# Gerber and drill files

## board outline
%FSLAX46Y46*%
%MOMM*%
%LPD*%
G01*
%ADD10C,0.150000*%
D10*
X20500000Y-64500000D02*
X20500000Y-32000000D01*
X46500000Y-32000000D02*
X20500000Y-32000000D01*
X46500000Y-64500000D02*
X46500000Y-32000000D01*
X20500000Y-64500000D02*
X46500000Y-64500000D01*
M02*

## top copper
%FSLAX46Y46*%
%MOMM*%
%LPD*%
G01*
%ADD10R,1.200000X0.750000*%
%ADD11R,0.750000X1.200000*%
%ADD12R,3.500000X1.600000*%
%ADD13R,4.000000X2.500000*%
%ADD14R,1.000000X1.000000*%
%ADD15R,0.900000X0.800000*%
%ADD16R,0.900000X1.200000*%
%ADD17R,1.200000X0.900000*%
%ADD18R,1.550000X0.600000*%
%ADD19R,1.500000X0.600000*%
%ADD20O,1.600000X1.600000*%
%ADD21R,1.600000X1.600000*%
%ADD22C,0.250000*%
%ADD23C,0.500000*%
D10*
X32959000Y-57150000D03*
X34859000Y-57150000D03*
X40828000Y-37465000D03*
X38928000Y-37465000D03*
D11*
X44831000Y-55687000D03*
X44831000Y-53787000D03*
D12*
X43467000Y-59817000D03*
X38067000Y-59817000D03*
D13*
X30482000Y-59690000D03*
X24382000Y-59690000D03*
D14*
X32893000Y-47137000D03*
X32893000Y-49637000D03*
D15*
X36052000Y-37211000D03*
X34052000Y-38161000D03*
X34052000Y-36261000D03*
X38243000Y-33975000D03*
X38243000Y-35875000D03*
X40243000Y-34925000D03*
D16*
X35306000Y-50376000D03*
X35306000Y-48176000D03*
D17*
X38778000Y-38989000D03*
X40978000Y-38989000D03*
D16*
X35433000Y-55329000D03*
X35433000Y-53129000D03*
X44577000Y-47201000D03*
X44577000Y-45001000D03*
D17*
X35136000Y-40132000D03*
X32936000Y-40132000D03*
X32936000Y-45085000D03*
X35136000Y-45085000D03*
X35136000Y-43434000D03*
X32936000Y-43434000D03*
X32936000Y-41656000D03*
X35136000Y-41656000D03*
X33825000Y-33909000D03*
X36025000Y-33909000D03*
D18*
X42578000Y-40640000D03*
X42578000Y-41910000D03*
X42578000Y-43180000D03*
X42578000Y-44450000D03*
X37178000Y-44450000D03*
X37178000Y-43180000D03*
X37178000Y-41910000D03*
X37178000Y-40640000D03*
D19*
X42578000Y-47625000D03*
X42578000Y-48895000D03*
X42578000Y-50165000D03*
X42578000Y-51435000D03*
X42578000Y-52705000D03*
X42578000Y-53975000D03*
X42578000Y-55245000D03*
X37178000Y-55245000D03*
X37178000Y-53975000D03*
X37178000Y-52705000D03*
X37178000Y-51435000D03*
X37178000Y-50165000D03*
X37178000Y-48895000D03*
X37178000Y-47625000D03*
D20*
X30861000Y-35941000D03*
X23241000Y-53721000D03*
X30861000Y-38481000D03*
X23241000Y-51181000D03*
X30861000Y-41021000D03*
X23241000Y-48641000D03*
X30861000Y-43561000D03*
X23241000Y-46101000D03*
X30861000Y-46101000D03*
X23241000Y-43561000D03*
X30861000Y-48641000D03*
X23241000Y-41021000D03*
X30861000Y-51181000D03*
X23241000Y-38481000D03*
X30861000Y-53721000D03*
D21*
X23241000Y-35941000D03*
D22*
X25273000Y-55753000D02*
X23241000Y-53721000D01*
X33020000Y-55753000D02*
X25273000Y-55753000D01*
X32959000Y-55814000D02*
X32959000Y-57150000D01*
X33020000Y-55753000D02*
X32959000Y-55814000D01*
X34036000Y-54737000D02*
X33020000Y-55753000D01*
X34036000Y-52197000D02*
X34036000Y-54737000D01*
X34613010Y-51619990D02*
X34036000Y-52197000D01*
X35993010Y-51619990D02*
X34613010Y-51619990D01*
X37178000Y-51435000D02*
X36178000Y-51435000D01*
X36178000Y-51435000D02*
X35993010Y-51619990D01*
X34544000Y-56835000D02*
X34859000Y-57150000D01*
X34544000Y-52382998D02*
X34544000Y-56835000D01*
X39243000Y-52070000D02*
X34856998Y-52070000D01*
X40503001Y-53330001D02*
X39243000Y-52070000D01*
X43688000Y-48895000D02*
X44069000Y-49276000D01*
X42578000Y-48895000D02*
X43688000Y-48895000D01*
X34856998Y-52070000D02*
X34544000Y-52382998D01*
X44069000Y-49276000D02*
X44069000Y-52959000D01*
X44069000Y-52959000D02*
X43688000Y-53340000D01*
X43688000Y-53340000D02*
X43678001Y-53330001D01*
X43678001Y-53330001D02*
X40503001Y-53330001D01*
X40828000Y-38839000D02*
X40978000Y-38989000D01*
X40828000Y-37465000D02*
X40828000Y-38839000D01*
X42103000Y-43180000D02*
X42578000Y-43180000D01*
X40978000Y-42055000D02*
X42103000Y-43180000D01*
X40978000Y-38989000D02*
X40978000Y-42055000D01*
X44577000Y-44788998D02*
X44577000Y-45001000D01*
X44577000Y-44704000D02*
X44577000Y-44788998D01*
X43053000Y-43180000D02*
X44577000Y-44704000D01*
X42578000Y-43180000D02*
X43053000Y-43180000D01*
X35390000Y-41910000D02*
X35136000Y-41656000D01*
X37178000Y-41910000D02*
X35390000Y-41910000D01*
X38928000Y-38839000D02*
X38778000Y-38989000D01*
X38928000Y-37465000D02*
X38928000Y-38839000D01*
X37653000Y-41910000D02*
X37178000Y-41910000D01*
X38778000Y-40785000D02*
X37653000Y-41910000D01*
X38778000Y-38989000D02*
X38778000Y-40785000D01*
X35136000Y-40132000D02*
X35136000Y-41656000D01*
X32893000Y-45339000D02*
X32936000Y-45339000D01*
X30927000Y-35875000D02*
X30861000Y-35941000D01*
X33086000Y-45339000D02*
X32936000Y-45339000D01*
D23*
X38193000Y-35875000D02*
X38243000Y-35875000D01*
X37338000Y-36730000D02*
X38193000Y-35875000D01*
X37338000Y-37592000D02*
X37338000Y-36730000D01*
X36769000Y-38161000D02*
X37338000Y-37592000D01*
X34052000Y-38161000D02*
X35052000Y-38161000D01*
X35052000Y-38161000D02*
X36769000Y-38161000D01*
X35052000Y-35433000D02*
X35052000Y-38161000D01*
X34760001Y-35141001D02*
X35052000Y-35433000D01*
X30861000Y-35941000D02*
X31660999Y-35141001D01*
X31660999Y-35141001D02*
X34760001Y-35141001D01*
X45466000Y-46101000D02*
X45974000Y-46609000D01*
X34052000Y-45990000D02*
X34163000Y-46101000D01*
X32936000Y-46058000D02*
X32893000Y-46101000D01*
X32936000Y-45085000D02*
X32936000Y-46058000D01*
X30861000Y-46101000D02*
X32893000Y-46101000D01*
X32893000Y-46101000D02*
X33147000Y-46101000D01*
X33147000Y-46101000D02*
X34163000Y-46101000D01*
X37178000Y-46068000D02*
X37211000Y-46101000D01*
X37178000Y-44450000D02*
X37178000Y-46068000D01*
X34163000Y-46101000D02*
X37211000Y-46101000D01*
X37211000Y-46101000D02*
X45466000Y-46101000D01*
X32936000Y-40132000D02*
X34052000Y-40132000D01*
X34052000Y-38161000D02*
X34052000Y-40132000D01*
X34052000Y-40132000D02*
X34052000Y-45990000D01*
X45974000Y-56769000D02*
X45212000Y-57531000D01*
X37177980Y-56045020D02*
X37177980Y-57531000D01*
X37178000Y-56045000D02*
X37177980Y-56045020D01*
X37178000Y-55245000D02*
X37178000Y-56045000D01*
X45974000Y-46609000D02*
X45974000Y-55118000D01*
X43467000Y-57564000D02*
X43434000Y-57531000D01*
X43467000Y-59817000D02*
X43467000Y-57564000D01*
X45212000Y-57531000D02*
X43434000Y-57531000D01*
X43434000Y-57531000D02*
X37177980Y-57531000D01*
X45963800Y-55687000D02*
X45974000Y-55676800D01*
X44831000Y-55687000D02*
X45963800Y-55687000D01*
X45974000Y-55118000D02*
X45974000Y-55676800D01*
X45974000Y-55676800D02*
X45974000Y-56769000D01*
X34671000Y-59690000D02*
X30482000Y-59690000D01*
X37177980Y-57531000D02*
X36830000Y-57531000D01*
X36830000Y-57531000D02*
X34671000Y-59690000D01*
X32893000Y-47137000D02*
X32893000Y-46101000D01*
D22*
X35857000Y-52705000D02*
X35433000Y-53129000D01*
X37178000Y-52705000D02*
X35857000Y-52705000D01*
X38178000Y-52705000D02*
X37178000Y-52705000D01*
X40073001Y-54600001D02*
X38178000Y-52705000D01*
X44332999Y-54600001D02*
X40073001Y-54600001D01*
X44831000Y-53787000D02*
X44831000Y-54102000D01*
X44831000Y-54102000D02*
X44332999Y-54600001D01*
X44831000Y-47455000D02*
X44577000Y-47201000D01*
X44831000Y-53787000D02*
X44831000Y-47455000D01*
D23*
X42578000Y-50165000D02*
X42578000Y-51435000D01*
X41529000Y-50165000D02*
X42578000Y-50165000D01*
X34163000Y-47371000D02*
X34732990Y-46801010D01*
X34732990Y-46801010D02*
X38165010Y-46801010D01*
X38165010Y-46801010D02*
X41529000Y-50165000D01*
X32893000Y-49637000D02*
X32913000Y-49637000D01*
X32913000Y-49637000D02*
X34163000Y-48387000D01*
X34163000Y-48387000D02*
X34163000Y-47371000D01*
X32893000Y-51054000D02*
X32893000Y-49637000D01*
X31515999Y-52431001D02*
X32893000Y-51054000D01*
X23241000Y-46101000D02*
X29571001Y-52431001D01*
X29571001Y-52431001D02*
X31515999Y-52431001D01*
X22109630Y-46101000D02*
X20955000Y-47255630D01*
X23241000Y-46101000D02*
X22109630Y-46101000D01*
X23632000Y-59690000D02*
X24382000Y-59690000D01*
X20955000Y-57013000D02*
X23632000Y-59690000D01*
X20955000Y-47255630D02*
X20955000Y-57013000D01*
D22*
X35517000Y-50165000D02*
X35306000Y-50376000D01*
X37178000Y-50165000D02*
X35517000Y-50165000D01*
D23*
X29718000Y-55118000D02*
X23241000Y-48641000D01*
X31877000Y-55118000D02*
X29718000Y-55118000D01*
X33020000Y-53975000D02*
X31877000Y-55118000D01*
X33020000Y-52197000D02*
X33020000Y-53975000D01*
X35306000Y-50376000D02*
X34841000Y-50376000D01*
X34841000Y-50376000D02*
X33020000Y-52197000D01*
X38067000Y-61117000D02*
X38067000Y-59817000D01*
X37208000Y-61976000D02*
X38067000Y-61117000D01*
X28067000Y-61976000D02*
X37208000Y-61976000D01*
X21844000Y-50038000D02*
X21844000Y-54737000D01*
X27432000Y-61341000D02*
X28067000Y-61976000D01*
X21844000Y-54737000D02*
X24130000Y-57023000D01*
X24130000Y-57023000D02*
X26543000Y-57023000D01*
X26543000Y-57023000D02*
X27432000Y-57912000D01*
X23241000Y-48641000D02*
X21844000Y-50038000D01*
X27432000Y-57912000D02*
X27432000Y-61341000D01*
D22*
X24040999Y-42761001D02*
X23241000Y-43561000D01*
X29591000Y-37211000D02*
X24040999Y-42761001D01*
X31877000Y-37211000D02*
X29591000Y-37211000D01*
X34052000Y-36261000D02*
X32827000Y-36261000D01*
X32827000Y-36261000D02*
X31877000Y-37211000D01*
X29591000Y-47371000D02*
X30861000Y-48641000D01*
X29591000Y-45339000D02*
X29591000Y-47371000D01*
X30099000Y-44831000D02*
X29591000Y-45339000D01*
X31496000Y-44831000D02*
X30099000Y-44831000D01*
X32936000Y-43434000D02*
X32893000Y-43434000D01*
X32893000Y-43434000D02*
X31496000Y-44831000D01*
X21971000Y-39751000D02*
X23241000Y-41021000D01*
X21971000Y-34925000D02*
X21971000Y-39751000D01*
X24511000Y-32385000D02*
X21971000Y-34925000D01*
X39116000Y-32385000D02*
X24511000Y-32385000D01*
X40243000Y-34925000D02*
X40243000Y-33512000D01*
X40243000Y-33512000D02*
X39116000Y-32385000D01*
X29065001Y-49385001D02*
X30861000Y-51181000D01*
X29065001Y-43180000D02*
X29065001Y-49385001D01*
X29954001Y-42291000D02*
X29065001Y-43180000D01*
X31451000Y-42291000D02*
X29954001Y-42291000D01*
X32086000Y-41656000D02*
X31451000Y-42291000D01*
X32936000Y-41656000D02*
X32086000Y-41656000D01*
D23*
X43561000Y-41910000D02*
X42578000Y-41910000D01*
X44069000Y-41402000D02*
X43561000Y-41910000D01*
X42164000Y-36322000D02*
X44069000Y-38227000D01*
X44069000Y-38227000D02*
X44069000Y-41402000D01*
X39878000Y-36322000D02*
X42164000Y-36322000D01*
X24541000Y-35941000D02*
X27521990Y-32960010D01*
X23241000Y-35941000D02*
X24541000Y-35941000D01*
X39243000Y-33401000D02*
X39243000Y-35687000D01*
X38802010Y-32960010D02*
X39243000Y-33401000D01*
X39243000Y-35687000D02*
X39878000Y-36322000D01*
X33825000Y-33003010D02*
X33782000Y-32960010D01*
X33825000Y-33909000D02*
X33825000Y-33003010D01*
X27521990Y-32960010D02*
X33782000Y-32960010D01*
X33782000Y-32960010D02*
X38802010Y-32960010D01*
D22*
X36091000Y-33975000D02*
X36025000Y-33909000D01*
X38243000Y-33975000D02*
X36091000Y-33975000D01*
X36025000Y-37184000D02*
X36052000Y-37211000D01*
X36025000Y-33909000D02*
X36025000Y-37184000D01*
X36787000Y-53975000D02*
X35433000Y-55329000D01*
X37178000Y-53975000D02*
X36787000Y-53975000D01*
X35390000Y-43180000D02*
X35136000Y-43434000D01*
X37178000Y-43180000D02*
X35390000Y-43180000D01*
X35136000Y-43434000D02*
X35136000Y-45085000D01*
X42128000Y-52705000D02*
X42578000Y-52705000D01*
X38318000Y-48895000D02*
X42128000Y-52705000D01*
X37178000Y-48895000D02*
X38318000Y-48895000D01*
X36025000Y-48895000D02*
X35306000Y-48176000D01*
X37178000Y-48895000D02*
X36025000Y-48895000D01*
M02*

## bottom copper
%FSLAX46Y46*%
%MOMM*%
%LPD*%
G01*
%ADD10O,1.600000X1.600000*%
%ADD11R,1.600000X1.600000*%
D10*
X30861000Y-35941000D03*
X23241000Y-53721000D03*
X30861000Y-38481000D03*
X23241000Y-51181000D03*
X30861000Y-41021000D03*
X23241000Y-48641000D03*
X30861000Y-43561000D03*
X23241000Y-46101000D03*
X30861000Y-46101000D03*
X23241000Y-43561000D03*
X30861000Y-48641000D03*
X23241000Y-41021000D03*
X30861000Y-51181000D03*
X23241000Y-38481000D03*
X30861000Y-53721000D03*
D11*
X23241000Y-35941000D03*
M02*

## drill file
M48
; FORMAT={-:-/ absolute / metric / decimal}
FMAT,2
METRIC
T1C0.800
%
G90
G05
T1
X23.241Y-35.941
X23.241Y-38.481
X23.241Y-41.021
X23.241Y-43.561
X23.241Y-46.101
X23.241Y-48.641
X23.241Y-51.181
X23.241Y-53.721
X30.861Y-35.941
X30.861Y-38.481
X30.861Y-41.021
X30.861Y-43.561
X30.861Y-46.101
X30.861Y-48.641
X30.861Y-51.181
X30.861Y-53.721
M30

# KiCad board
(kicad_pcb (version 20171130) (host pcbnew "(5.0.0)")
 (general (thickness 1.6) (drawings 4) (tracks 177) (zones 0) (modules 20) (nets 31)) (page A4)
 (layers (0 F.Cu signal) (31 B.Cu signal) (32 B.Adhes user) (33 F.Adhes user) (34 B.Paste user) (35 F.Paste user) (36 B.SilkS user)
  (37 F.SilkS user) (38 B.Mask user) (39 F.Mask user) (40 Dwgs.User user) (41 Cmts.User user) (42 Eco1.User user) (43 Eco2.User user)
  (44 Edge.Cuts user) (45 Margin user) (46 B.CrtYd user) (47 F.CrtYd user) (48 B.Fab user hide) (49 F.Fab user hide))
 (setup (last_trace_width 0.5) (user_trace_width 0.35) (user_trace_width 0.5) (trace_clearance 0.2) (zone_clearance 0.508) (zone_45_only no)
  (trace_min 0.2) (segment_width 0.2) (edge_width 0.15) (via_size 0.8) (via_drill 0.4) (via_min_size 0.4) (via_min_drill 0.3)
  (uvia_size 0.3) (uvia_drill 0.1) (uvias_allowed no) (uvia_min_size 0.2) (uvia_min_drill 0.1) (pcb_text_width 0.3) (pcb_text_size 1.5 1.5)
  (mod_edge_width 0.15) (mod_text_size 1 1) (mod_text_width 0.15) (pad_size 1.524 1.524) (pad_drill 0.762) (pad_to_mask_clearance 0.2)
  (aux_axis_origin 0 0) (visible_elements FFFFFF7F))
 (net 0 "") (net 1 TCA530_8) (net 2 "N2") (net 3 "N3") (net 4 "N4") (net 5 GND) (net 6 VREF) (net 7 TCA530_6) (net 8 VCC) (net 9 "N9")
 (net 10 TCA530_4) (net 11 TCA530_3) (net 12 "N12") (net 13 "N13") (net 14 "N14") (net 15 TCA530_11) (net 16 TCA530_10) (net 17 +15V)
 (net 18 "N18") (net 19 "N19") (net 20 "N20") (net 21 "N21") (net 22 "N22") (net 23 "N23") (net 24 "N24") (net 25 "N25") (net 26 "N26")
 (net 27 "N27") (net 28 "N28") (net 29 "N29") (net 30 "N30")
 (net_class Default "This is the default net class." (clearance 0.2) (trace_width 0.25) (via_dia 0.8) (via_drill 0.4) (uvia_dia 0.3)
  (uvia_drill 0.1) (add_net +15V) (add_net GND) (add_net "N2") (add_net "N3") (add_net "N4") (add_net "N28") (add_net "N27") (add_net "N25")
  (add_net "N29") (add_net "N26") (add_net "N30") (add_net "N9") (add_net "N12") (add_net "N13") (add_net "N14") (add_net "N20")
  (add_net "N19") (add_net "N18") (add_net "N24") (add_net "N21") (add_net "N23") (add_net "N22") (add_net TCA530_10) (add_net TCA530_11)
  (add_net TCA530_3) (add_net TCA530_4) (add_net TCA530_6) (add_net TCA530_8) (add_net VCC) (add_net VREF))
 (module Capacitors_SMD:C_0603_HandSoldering (layer F.Cu) (at 33.909 57.15 180)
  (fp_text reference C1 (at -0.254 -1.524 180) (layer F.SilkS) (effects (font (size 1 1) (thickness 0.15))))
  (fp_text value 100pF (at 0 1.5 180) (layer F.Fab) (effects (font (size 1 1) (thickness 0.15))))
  (pad 2 smd rect (at 0.95 0 180) (size 1.2 0.75) (layers F.Cu F.Paste F.Mask) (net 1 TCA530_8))
  (pad 1 smd rect (at -0.95 0 180) (size 1.2 0.75) (layers F.Cu F.Paste F.Mask) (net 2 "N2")))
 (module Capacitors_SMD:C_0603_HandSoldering (layer F.Cu) (at 39.878 37.465 180)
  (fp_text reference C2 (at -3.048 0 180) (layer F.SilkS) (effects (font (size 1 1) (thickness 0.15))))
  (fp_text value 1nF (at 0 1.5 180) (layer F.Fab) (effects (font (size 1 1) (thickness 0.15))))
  (pad 1 smd rect (at -0.95 0 180) (size 1.2 0.75) (layers F.Cu F.Paste F.Mask) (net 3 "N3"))
  (pad 2 smd rect (at 0.95 0 180) (size 1.2 0.75) (layers F.Cu F.Paste F.Mask) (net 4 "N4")))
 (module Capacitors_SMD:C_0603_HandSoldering (layer F.Cu) (at 44.831 54.737 270)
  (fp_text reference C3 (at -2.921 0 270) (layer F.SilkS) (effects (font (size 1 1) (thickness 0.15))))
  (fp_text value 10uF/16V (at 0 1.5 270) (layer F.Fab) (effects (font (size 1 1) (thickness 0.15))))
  (pad 2 smd rect (at 0.95 0 270) (size 1.2 0.75) (layers F.Cu F.Paste F.Mask) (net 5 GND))
  (pad 1 smd rect (at -0.95 0 270) (size 1.2 0.75) (layers F.Cu F.Paste F.Mask) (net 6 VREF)))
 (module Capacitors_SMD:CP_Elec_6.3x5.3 (layer F.Cu) (at 40.767 59.817)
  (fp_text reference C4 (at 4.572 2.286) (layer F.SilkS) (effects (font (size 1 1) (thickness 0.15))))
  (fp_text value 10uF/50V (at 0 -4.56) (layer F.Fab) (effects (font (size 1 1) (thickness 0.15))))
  (pad 2 smd rect (at 2.7 0 180) (size 3.5 1.6) (layers F.Cu F.Paste F.Mask) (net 5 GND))
  (pad 1 smd rect (at -2.7 0 180) (size 3.5 1.6) (layers F.Cu F.Paste F.Mask) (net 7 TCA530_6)))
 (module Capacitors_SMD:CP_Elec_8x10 (layer F.Cu) (at 27.432 59.69)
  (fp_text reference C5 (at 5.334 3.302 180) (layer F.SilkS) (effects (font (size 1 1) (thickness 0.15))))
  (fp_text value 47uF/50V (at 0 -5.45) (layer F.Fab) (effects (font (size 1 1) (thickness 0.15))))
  (pad 2 smd rect (at 3.05 0 180) (size 4 2.5) (layers F.Cu F.Paste F.Mask) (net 5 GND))
  (pad 1 smd rect (at -3.05 0 180) (size 4 2.5) (layers F.Cu F.Paste F.Mask) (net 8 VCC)))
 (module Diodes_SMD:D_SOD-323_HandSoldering (layer F.Cu) (at 32.893 48.387 90)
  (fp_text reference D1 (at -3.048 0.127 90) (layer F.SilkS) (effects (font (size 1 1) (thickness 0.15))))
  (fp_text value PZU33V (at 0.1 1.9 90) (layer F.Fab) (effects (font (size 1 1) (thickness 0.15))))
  (pad 2 smd rect (at 1.25 0 90) (size 1 1) (layers F.Cu F.Paste F.Mask) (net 5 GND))
  (pad 1 smd rect (at -1.25 0 90) (size 1 1) (layers F.Cu F.Paste F.Mask) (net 8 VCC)))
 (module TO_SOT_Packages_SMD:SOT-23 (layer F.Cu) (at 35.052 37.211)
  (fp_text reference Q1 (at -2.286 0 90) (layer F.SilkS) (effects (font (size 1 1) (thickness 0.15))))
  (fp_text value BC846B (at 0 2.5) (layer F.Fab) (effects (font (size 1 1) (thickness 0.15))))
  (pad 3 smd rect (at 1 0) (size 0.9 0.8) (layers F.Cu F.Paste F.Mask) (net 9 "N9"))
  (pad 2 smd rect (at -1 0.95) (size 0.9 0.8) (layers F.Cu F.Paste F.Mask) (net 5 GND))
  (pad 1 smd rect (at -1 -0.95) (size 0.9 0.8) (layers F.Cu F.Paste F.Mask) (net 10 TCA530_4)))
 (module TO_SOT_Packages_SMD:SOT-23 (layer F.Cu) (at 39.243 34.925)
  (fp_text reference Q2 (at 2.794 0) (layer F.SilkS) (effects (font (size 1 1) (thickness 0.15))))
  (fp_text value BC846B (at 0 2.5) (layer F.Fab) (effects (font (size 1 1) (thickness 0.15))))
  (pad 1 smd rect (at -1 -0.95) (size 0.9 0.8) (layers F.Cu F.Paste F.Mask) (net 9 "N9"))
  (pad 2 smd rect (at -1 0.95) (size 0.9 0.8) (layers F.Cu F.Paste F.Mask) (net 5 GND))
  (pad 3 smd rect (at 1 0) (size 0.9 0.8) (layers F.Cu F.Paste F.Mask) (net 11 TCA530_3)))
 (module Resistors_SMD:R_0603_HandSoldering (layer F.Cu) (at 35.306 49.276 270)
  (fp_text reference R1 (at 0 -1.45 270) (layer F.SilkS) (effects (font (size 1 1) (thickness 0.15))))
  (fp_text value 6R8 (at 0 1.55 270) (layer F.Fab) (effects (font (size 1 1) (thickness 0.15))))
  (pad 2 smd rect (at 1.1 0 270) (size 1.2 0.9) (layers F.Cu F.Paste F.Mask) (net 7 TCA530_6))
  (pad 1 smd rect (at -1.1 0 270) (size 1.2 0.9) (layers F.Cu F.Paste F.Mask) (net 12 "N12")))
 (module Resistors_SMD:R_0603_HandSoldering (layer F.Cu) (at 39.878 38.989 180)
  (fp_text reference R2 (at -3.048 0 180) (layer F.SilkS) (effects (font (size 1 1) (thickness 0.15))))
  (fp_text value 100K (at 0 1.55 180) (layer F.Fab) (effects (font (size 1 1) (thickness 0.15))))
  (pad 2 smd rect (at 1.1 0 180) (size 1.2 0.9) (layers F.Cu F.Paste F.Mask) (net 4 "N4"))
  (pad 1 smd rect (at -1.1 0 180) (size 1.2 0.9) (layers F.Cu F.Paste F.Mask) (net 3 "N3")))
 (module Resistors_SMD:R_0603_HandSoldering (layer F.Cu) (at 35.433 54.229 270)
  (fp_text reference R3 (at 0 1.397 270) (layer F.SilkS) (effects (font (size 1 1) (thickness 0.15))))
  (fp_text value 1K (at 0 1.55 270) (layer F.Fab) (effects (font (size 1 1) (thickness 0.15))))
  (pad 2 smd rect (at 1.1 0 270) (size 1.2 0.9) (layers F.Cu F.Paste F.Mask) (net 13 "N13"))
  (pad 1 smd rect (at -1.1 0 270) (size 1.2 0.9) (layers F.Cu F.Paste F.Mask) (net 6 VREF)))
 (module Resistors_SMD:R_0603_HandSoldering (layer F.Cu) (at 44.577 46.101 90)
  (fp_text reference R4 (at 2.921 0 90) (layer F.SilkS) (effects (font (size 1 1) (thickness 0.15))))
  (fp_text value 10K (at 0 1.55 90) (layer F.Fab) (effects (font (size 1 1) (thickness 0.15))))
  (pad 1 smd rect (at -1.1 0 90) (size 1.2 0.9) (layers F.Cu F.Paste F.Mask) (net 6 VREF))
  (pad 2 smd rect (at 1.1 0 90) (size 1.2 0.9) (layers F.Cu F.Paste F.Mask) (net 3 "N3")))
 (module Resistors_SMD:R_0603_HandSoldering (layer F.Cu) (at 34.036 40.132 180)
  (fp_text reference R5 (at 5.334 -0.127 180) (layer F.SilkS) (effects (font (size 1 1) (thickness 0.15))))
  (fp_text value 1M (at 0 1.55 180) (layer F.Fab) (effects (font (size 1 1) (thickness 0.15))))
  (pad 1 smd rect (at -1.1 0 180) (size 1.2 0.9) (layers F.Cu F.Paste F.Mask) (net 4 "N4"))
  (pad 2 smd rect (at 1.1 0 180) (size 1.2 0.9) (layers F.Cu F.Paste F.Mask) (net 5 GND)))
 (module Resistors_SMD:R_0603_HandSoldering (layer F.Cu) (at 34.036 45.085 180)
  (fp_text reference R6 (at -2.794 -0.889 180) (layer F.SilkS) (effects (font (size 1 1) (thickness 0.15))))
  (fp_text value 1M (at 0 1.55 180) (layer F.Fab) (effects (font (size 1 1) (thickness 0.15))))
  (pad 2 smd rect (at 1.1 0 180) (size 1.2 0.9) (layers F.Cu F.Paste F.Mask) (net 5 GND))
  (pad 1 smd rect (at -1.1 0 180) (size 1.2 0.9) (layers F.Cu F.Paste F.Mask) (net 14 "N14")))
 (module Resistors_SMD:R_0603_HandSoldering (layer F.Cu) (at 34.036 43.434 180)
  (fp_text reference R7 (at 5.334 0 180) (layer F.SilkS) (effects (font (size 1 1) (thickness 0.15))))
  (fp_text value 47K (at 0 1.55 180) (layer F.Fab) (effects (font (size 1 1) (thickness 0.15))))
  (pad 1 smd rect (at -1.1 0 180) (size 1.2 0.9) (layers F.Cu F.Paste F.Mask) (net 14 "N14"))
  (pad 2 smd rect (at 1.1 0 180) (size 1.2 0.9) (layers F.Cu F.Paste F.Mask) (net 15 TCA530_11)))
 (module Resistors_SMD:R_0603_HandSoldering (layer F.Cu) (at 34.036 41.656 180)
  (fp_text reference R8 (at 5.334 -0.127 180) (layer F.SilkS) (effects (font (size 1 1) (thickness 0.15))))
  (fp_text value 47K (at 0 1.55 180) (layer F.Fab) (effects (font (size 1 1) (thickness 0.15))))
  (pad 2 smd rect (at 1.1 0 180) (size 1.2 0.9) (layers F.Cu F.Paste F.Mask) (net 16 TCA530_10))
  (pad 1 smd rect (at -1.1 0 180) (size 1.2 0.9) (layers F.Cu F.Paste F.Mask) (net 4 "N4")))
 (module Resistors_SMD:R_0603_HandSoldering (layer F.Cu) (at 34.925 33.909)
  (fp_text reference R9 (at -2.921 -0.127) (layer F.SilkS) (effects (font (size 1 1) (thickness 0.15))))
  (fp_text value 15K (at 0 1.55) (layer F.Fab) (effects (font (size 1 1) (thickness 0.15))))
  (pad 1 smd rect (at -1.1 0) (size 1.2 0.9) (layers F.Cu F.Paste F.Mask) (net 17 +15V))
  (pad 2 smd rect (at 1.1 0) (size 1.2 0.9) (layers F.Cu F.Paste F.Mask) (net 9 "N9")))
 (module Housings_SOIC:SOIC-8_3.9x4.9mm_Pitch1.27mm (layer F.Cu) (at 39.878 42.545)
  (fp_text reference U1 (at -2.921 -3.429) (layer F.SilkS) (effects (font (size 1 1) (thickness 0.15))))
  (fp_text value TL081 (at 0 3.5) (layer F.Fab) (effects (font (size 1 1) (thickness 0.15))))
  (pad 8 smd rect (at 2.7 -1.905) (size 1.55 0.6) (layers F.Cu F.Paste F.Mask) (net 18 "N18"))
  (pad 7 smd rect (at 2.7 -0.635) (size 1.55 0.6) (layers F.Cu F.Paste F.Mask) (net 17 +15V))
  (pad 6 smd rect (at 2.7 0.635) (size 1.55 0.6) (layers F.Cu F.Paste F.Mask) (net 3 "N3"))
  (pad 5 smd rect (at 2.7 1.905) (size 1.55 0.6) (layers F.Cu F.Paste F.Mask) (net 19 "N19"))
  (pad 4 smd rect (at -2.7 1.905) (size 1.55 0.6) (layers F.Cu F.Paste F.Mask) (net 5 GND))
  (pad 3 smd rect (at -2.7 0.635) (size 1.55 0.6) (layers F.Cu F.Paste F.Mask) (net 14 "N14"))
  (pad 2 smd rect (at -2.7 -0.635) (size 1.55 0.6) (layers F.Cu F.Paste F.Mask) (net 4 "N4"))
  (pad 1 smd rect (at -2.7 -1.905) (size 1.55 0.6) (layers F.Cu F.Paste F.Mask) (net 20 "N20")))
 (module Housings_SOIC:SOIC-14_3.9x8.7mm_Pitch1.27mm (layer F.Cu) (at 39.878 51.435)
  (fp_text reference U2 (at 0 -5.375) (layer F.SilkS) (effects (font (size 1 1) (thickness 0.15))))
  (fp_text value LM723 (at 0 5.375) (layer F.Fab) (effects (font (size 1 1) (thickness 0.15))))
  (pad 14 smd rect (at 2.7 -3.81) (size 1.5 0.6) (layers F.Cu F.Paste F.Mask) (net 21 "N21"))
  (pad 13 smd rect (at 2.7 -2.54) (size 1.5 0.6) (layers F.Cu F.Paste F.Mask) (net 2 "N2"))
  (pad 12 smd rect (at 2.7 -1.27) (size 1.5 0.6) (layers F.Cu F.Paste F.Mask) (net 8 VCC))
  (pad 11 smd rect (at 2.7 0) (size 1.5 0.6) (layers F.Cu F.Paste F.Mask) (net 8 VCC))
  (pad 10 smd rect (at 2.7 1.27) (size 1.5 0.6) (layers F.Cu F.Paste F.Mask) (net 12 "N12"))
  (pad 9 smd rect (at 2.7 2.54) (size 1.5 0.6) (layers F.Cu F.Paste F.Mask) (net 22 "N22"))
  (pad 8 smd rect (at 2.7 3.81) (size 1.5 0.6) (layers F.Cu F.Paste F.Mask) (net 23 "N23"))
  (pad 7 smd rect (at -2.7 3.81) (size 1.5 0.6) (layers F.Cu F.Paste F.Mask) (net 5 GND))
  (pad 6 smd rect (at -2.7 2.54) (size 1.5 0.6) (layers F.Cu F.Paste F.Mask) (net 13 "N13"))
  (pad 5 smd rect (at -2.7 1.27) (size 1.5 0.6) (layers F.Cu F.Paste F.Mask) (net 6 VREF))
  (pad 4 smd rect (at -2.7 0) (size 1.5 0.6) (layers F.Cu F.Paste F.Mask) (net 1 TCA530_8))
  (pad 3 smd rect (at -2.7 -1.27) (size 1.5 0.6) (layers F.Cu F.Paste F.Mask) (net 7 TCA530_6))
  (pad 2 smd rect (at -2.7 -2.54) (size 1.5 0.6) (layers F.Cu F.Paste F.Mask) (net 12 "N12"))
  (pad 1 smd rect (at -2.7 -3.81) (size 1.5 0.6) (layers F.Cu F.Paste F.Mask) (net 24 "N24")))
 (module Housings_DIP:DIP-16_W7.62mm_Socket (layer F.Cu) (at 23.241 35.941)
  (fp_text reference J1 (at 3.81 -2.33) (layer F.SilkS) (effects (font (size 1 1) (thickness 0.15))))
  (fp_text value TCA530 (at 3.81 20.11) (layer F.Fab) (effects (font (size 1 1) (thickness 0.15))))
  (pad 16 thru_hole oval (at 7.62 0) (size 1.6 1.6) (drill 0.8) (layers *.Cu *.Mask) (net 5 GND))
  (pad 8 thru_hole oval (at 0 17.78) (size 1.6 1.6) (drill 0.8) (layers *.Cu *.Mask) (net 1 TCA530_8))
  (pad 15 thru_hole oval (at 7.62 2.54) (size 1.6 1.6) (drill 0.8) (layers *.Cu *.Mask) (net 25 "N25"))
  (pad 7 thru_hole oval (at 0 15.24) (size 1.6 1.6) (drill 0.8) (layers *.Cu *.Mask) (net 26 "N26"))
  (pad 14 thru_hole oval (at 7.62 5.08) (size 1.6 1.6) (drill 0.8) (layers *.Cu *.Mask) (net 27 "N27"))
  (pad 6 thru_hole oval (at 0 12.7) (size 1.6 1.6) (drill 0.8) (layers *.Cu *.Mask) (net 7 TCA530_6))
  (pad 13 thru_hole oval (at 7.62 7.62) (size 1.6 1.6) (drill 0.8) (layers *.Cu *.Mask) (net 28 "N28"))
  (pad 5 thru_hole oval (at 0 10.16) (size 1.6 1.6) (drill 0.8) (layers *.Cu *.Mask) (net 8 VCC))
  (pad 12 thru_hole oval (at 7.62 10.16) (size 1.6 1.6) (drill 0.8) (layers *.Cu *.Mask) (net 5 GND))
  (pad 4 thru_hole oval (at 0 7.62) (size 1.6 1.6) (drill 0.8) (layers *.Cu *.Mask) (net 10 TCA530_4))
  (pad 11 thru_hole oval (at 7.62 12.7) (size 1.6 1.6) (drill 0.8) (layers *.Cu *.Mask) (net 15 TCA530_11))
  (pad 3 thru_hole oval (at 0 5.08) (size 1.6 1.6) (drill 0.8) (layers *.Cu *.Mask) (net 11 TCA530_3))
  (pad 10 thru_hole oval (at 7.62 15.24) (size 1.6 1.6) (drill 0.8) (layers *.Cu *.Mask) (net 16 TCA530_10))
  (pad 2 thru_hole oval (at 0 2.54) (size 1.6 1.6) (drill 0.8) (layers *.Cu *.Mask) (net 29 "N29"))
  (pad 9 thru_hole oval (at 7.62 17.78) (size 1.6 1.6) (drill 0.8) (layers *.Cu *.Mask) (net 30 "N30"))
  (pad 1 thru_hole rect (at 0 0) (size 1.6 1.6) (drill 0.8) (layers *.Cu *.Mask) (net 17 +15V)))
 (gr_line (start 20.5 64.5) (end 20.5 32) (layer Edge.Cuts) (width 0.15))
 (gr_line (start 46.5 32) (end 20.5 32) (layer Edge.Cuts) (width 0.15))
 (gr_line (start 46.5 64.5) (end 46.5 32) (layer Edge.Cuts) (width 0.15))
 (gr_line (start 20.5 64.5) (end 46.5 64.5) (layer Edge.Cuts) (width 0.15))
 (segment (start 25.273 55.753) (end 23.241 53.721) (width 0.25) (layer F.Cu) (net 1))
 (segment (start 33.02 55.753) (end 25.273 55.753) (width 0.25) (layer F.Cu) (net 1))
 (segment (start 32.959 55.814) (end 32.959 57.15) (width 0.25) (layer F.Cu) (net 1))
 (segment (start 33.02 55.753) (end 32.959 55.814) (width 0.25) (layer F.Cu) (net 1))
 (segment (start 34.036 54.737) (end 33.02 55.753) (width 0.25) (layer F.Cu) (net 1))
 (segment (start 34.036 52.197) (end 34.036 54.737) (width 0.25) (layer F.Cu) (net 1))
 (segment (start 34.61301 51.61999) (end 34.036 52.197) (width 0.25) (layer F.Cu) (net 1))
 (segment (start 35.99301 51.61999) (end 34.61301 51.61999) (width 0.25) (layer F.Cu) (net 1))
 (segment (start 37.178 51.435) (end 36.178 51.435) (width 0.25) (layer F.Cu) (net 1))
 (segment (start 36.178 51.435) (end 35.99301 51.61999) (width 0.25) (layer F.Cu) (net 1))
 (segment (start 34.544 56.835) (end 34.859 57.15) (width 0.25) (layer F.Cu) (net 2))
 (segment (start 34.544 52.382998) (end 34.544 56.835) (width 0.25) (layer F.Cu) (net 2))
 (segment (start 39.243 52.07) (end 34.856998 52.07) (width 0.25) (layer F.Cu) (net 2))
 (segment (start 40.503001 53.330001) (end 39.243 52.07) (width 0.25) (layer F.Cu) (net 2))
 (segment (start 43.688 48.895) (end 44.069 49.276) (width 0.25) (layer F.Cu) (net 2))
 (segment (start 42.578 48.895) (end 43.688 48.895) (width 0.25) (layer F.Cu) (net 2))
 (segment (start 34.856998 52.07) (end 34.544 52.382998) (width 0.25) (layer F.Cu) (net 2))
 (segment (start 44.069 49.276) (end 44.069 52.959) (width 0.25) (layer F.Cu) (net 2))
 (segment (start 44.069 52.959) (end 43.688 53.34) (width 0.25) (layer F.Cu) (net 2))
 (segment (start 43.688 53.34) (end 43.678001 53.330001) (width 0.25) (layer F.Cu) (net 2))
 (segment (start 43.678001 53.330001) (end 40.503001 53.330001) (width 0.25) (layer F.Cu) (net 2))
 (segment (start 40.828 38.839) (end 40.978 38.989) (width 0.25) (layer F.Cu) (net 3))
 (segment (start 40.828 37.465) (end 40.828 38.839) (width 0.25) (layer F.Cu) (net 3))
 (segment (start 42.103 43.18) (end 42.578 43.18) (width 0.25) (layer F.Cu) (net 3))
 (segment (start 40.978 42.055) (end 42.103 43.18) (width 0.25) (layer F.Cu) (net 3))
 (segment (start 40.978 38.989) (end 40.978 42.055) (width 0.25) (layer F.Cu) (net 3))
 (segment (start 44.577 44.788998) (end 44.577 45.001) (width 0.25) (layer F.Cu) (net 3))
 (segment (start 44.577 44.704) (end 44.577 44.788998) (width 0.25) (layer F.Cu) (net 3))
 (segment (start 43.053 43.18) (end 44.577 44.704) (width 0.25) (layer F.Cu) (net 3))
 (segment (start 42.578 43.18) (end 43.053 43.18) (width 0.25) (layer F.Cu) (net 3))
 (segment (start 35.39 41.91) (end 35.136 41.656) (width 0.25) (layer F.Cu) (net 4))
 (segment (start 37.178 41.91) (end 35.39 41.91) (width 0.25) (layer F.Cu) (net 4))
 (segment (start 38.928 38.839) (end 38.778 38.989) (width 0.25) (layer F.Cu) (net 4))
 (segment (start 38.928 37.465) (end 38.928 38.839) (width 0.25) (layer F.Cu) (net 4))
 (segment (start 37.653 41.91) (end 37.178 41.91) (width 0.25) (layer F.Cu) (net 4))
 (segment (start 38.778 40.785) (end 37.653 41.91) (width 0.25) (layer F.Cu) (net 4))
 (segment (start 38.778 38.989) (end 38.778 40.785) (width 0.25) (layer F.Cu) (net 4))
 (segment (start 35.136 40.132) (end 35.136 41.656) (width 0.25) (layer F.Cu) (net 4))
 (segment (start 32.893 45.339) (end 32.936 45.339) (width 0.25) (layer F.Cu) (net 5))
 (segment (start 30.927 35.875) (end 30.861 35.941) (width 0.25) (layer F.Cu) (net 5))
 (segment (start 33.086 45.339) (end 32.936 45.339) (width 0.25) (layer F.Cu) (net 5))
 (segment (start 38.193 35.875) (end 38.243 35.875) (width 0.5) (layer F.Cu) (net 5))
 (segment (start 37.338 36.73) (end 38.193 35.875) (width 0.5) (layer F.Cu) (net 5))
 (segment (start 37.338 37.592) (end 37.338 36.73) (width 0.5) (layer F.Cu) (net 5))
 (segment (start 36.769 38.161) (end 37.338 37.592) (width 0.5) (layer F.Cu) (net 5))
 (segment (start 34.052 38.161) (end 35.052 38.161) (width 0.5) (layer F.Cu) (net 5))
 (segment (start 35.052 38.161) (end 36.769 38.161) (width 0.5) (layer F.Cu) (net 5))
 (segment (start 35.052 35.433) (end 35.052 38.161) (width 0.5) (layer F.Cu) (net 5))
 (segment (start 34.760001 35.141001) (end 35.052 35.433) (width 0.5) (layer F.Cu) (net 5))
 (segment (start 30.861 35.941) (end 31.660999 35.141001) (width 0.5) (layer F.Cu) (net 5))
 (segment (start 31.660999 35.141001) (end 34.760001 35.141001) (width 0.5) (layer F.Cu) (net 5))
 (segment (start 45.466 46.101) (end 45.974 46.609) (width 0.5) (layer F.Cu) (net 5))
 (segment (start 34.052 45.99) (end 34.163 46.101) (width 0.5) (layer F.Cu) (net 5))
 (segment (start 32.936 46.058) (end 32.893 46.101) (width 0.5) (layer F.Cu) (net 5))
 (segment (start 32.936 45.085) (end 32.936 46.058) (width 0.5) (layer F.Cu) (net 5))
 (segment (start 30.861 46.101) (end 32.893 46.101) (width 0.5) (layer F.Cu) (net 5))
 (segment (start 32.893 46.101) (end 33.147 46.101) (width 0.5) (layer F.Cu) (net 5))
 (segment (start 33.147 46.101) (end 34.163 46.101) (width 0.5) (layer F.Cu) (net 5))
 (segment (start 37.178 46.068) (end 37.211 46.101) (width 0.5) (layer F.Cu) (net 5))
 (segment (start 37.178 44.45) (end 37.178 46.068) (width 0.5) (layer F.Cu) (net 5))
 (segment (start 34.163 46.101) (end 37.211 46.101) (width 0.5) (layer F.Cu) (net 5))
 (segment (start 37.211 46.101) (end 45.466 46.101) (width 0.5) (layer F.Cu) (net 5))
 (segment (start 32.936 40.132) (end 34.052 40.132) (width 0.5) (layer F.Cu) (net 5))
 (segment (start 34.052 38.161) (end 34.052 40.132) (width 0.5) (layer F.Cu) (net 5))
 (segment (start 34.052 40.132) (end 34.052 45.99) (width 0.5) (layer F.Cu) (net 5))
 (segment (start 45.974 56.769) (end 45.212 57.531) (width 0.5) (layer F.Cu) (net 5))
 (segment (start 37.17798 56.04502) (end 37.17798 57.531) (width 0.5) (layer F.Cu) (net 5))
 (segment (start 37.178 56.045) (end 37.17798 56.04502) (width 0.5) (layer F.Cu) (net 5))
 (segment (start 37.178 55.245) (end 37.178 56.045) (width 0.5) (layer F.Cu) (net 5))
 (segment (start 45.974 46.609) (end 45.974 55.118) (width 0.5) (layer F.Cu) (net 5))
 (segment (start 43.467 57.564) (end 43.434 57.531) (width 0.5) (layer F.Cu) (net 5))
 (segment (start 43.467 59.817) (end 43.467 57.564) (width 0.5) (layer F.Cu) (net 5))
 (segment (start 45.212 57.531) (end 43.434 57.531) (width 0.5) (layer F.Cu) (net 5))
 (segment (start 43.434 57.531) (end 37.17798 57.531) (width 0.5) (layer F.Cu) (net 5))
 (segment (start 45.9638 55.687) (end 45.974 55.6768) (width 0.5) (layer F.Cu) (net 5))
 (segment (start 44.831 55.687) (end 45.9638 55.687) (width 0.5) (layer F.Cu) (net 5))
 (segment (start 45.974 55.118) (end 45.974 55.6768) (width 0.5) (layer F.Cu) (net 5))
 (segment (start 45.974 55.6768) (end 45.974 56.769) (width 0.5) (layer F.Cu) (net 5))
 (segment (start 34.671 59.69) (end 30.482 59.69) (width 0.5) (layer F.Cu) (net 5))
 (segment (start 37.17798 57.531) (end 36.83 57.531) (width 0.5) (layer F.Cu) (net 5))
 (segment (start 36.83 57.531) (end 34.671 59.69) (width 0.5) (layer F.Cu) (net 5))
 (segment (start 32.893 47.137) (end 32.893 46.101) (width 0.5) (layer F.Cu) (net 5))
 (segment (start 35.857 52.705) (end 35.433 53.129) (width 0.25) (layer F.Cu) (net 6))
 (segment (start 37.178 52.705) (end 35.857 52.705) (width 0.25) (layer F.Cu) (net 6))
 (segment (start 38.178 52.705) (end 37.178 52.705) (width 0.25) (layer F.Cu) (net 6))
 (segment (start 40.073001 54.600001) (end 38.178 52.705) (width 0.25) (layer F.Cu) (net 6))
 (segment (start 44.332999 54.600001) (end 40.073001 54.600001) (width 0.25) (layer F.Cu) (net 6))
 (segment (start 44.831 53.787) (end 44.831 54.102) (width 0.25) (layer F.Cu) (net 6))
 (segment (start 44.831 54.102) (end 44.332999 54.600001) (width 0.25) (layer F.Cu) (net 6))
 (segment (start 44.831 47.455) (end 44.577 47.201) (width 0.25) (layer F.Cu) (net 6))
 (segment (start 44.831 53.787) (end 44.831 47.455) (width 0.25) (layer F.Cu) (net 6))
 (segment (start 42.578 50.165) (end 42.578 51.435) (width 0.5) (layer F.Cu) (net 8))
 (segment (start 41.529 50.165) (end 42.578 50.165) (width 0.5) (layer F.Cu) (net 8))
 (segment (start 34.163 47.371) (end 34.73299 46.80101) (width 0.5) (layer F.Cu) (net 8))
 (segment (start 34.73299 46.80101) (end 38.16501 46.80101) (width 0.5) (layer F.Cu) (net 8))
 (segment (start 38.16501 46.80101) (end 41.529 50.165) (width 0.5) (layer F.Cu) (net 8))
 (segment (start 32.893 49.637) (end 32.913 49.637) (width 0.5) (layer F.Cu) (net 8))
 (segment (start 32.913 49.637) (end 34.163 48.387) (width 0.5) (layer F.Cu) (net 8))
 (segment (start 34.163 48.387) (end 34.163 47.371) (width 0.5) (layer F.Cu) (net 8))
 (segment (start 32.893 51.054) (end 32.893 49.637) (width 0.5) (layer F.Cu) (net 8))
 (segment (start 31.515999 52.431001) (end 32.893 51.054) (width 0.5) (layer F.Cu) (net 8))
 (segment (start 23.241 46.101) (end 29.571001 52.431001) (width 0.5) (layer F.Cu) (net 8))
 (segment (start 29.571001 52.431001) (end 31.515999 52.431001) (width 0.5) (layer F.Cu) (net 8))
 (segment (start 22.10963 46.101) (end 20.955 47.25563) (width 0.5) (layer F.Cu) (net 8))
 (segment (start 23.241 46.101) (end 22.10963 46.101) (width 0.5) (layer F.Cu) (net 8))
 (segment (start 23.632 59.69) (end 24.382 59.69) (width 0.5) (layer F.Cu) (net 8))
 (segment (start 20.955 57.013) (end 23.632 59.69) (width 0.5) (layer F.Cu) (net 8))
 (segment (start 20.955 47.25563) (end 20.955 57.013) (width 0.5) (layer F.Cu) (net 8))
 (segment (start 35.517 50.165) (end 35.306 50.376) (width 0.25) (layer F.Cu) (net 7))
 (segment (start 37.178 50.165) (end 35.517 50.165) (width 0.25) (layer F.Cu) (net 7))
 (segment (start 29.718 55.118) (end 23.241 48.641) (width 0.5) (layer F.Cu) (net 7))
 (segment (start 31.877 55.118) (end 29.718 55.118) (width 0.5) (layer F.Cu) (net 7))
 (segment (start 33.02 53.975) (end 31.877 55.118) (width 0.5) (layer F.Cu) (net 7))
 (segment (start 33.02 52.197) (end 33.02 53.975) (width 0.5) (layer F.Cu) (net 7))
 (segment (start 35.306 50.376) (end 34.841 50.376) (width 0.5) (layer F.Cu) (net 7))
 (segment (start 34.841 50.376) (end 33.02 52.197) (width 0.5) (layer F.Cu) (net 7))
 (segment (start 38.067 61.117) (end 38.067 59.817) (width 0.5) (layer F.Cu) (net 7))
 (segment (start 37.208 61.976) (end 38.067 61.117) (width 0.5) (layer F.Cu) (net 7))
 (segment (start 28.067 61.976) (end 37.208 61.976) (width 0.5) (layer F.Cu) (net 7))
 (segment (start 21.844 50.038) (end 21.844 54.737) (width 0.5) (layer F.Cu) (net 7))
 (segment (start 27.432 61.341) (end 28.067 61.976) (width 0.5) (layer F.Cu) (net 7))
 (segment (start 21.844 54.737) (end 24.13 57.023) (width 0.5) (layer F.Cu) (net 7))
 (segment (start 24.13 57.023) (end 26.543 57.023) (width 0.5) (layer F.Cu) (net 7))
 (segment (start 26.543 57.023) (end 27.432 57.912) (width 0.5) (layer F.Cu) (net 7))
 (segment (start 23.241 48.641) (end 21.844 50.038) (width 0.5) (layer F.Cu) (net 7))
 (segment (start 27.432 57.912) (end 27.432 61.341) (width 0.5) (layer F.Cu) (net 7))
 (segment (start 24.040999 42.761001) (end 23.241 43.561) (width 0.25) (layer F.Cu) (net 10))
 (segment (start 29.591 37.211) (end 24.040999 42.761001) (width 0.25) (layer F.Cu) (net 10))
 (segment (start 31.877 37.211) (end 29.591 37.211) (width 0.25) (layer F.Cu) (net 10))
 (segment (start 34.052 36.261) (end 32.827 36.261) (width 0.25) (layer F.Cu) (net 10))
 (segment (start 32.827 36.261) (end 31.877 37.211) (width 0.25) (layer F.Cu) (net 10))
 (segment (start 29.591 47.371) (end 30.861 48.641) (width 0.25) (layer F.Cu) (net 15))
 (segment (start 29.591 45.339) (end 29.591 47.371) (width 0.25) (layer F.Cu) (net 15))
 (segment (start 30.099 44.831) (end 29.591 45.339) (width 0.25) (layer F.Cu) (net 15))
 (segment (start 31.496 44.831) (end 30.099 44.831) (width 0.25) (layer F.Cu) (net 15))
 (segment (start 32.936 43.434) (end 32.893 43.434) (width 0.25) (layer F.Cu) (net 15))
 (segment (start 32.893 43.434) (end 31.496 44.831) (width 0.25) (layer F.Cu) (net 15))
 (segment (start 21.971 39.751) (end 23.241 41.021) (width 0.25) (layer F.Cu) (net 11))
 (segment (start 21.971 34.925) (end 21.971 39.751) (width 0.25) (layer F.Cu) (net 11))
 (segment (start 24.511 32.385) (end 21.971 34.925) (width 0.25) (layer F.Cu) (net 11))
 (segment (start 39.116 32.385) (end 24.511 32.385) (width 0.25) (layer F.Cu) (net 11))
 (segment (start 40.243 34.925) (end 40.243 33.512) (width 0.25) (layer F.Cu) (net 11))
 (segment (start 40.243 33.512) (end 39.116 32.385) (width 0.25) (layer F.Cu) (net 11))
 (segment (start 29.065001 49.385001) (end 30.861 51.181) (width 0.25) (layer F.Cu) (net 16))
 (segment (start 29.065001 43.18) (end 29.065001 49.385001) (width 0.25) (layer F.Cu) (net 16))
 (segment (start 29.954001 42.291) (end 29.065001 43.18) (width 0.25) (layer F.Cu) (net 16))
 (segment (start 31.451 42.291) (end 29.954001 42.291) (width 0.25) (layer F.Cu) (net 16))
 (segment (start 32.086 41.656) (end 31.451 42.291) (width 0.25) (layer F.Cu) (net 16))
 (segment (start 32.936 41.656) (end 32.086 41.656) (width 0.25) (layer F.Cu) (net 16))
 (segment (start 43.561 41.91) (end 42.578 41.91) (width 0.5) (layer F.Cu) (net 17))
 (segment (start 44.069 41.402) (end 43.561 41.91) (width 0.5) (layer F.Cu) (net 17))
 (segment (start 42.164 36.322) (end 44.069 38.227) (width 0.5) (layer F.Cu) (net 17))
 (segment (start 44.069 38.227) (end 44.069 41.402) (width 0.5) (layer F.Cu) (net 17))
 (segment (start 39.878 36.322) (end 42.164 36.322) (width 0.5) (layer F.Cu) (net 17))
 (segment (start 24.541 35.941) (end 27.52199 32.96001) (width 0.5) (layer F.Cu) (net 17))
 (segment (start 23.241 35.941) (end 24.541 35.941) (width 0.5) (layer F.Cu) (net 17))
 (segment (start 39.243 33.401) (end 39.243 35.687) (width 0.5) (layer F.Cu) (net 17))
 (segment (start 38.80201 32.96001) (end 39.243 33.401) (width 0.5) (layer F.Cu) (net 17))
 (segment (start 39.243 35.687) (end 39.878 36.322) (width 0.5) (layer F.Cu) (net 17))
 (segment (start 33.825 33.00301) (end 33.782 32.96001) (width 0.5) (layer F.Cu) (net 17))
 (segment (start 33.825 33.909) (end 33.825 33.00301) (width 0.5) (layer F.Cu) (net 17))
 (segment (start 27.52199 32.96001) (end 33.782 32.96001) (width 0.5) (layer F.Cu) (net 17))
 (segment (start 33.782 32.96001) (end 38.80201 32.96001) (width 0.5) (layer F.Cu) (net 17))
 (segment (start 36.091 33.975) (end 36.025 33.909) (width 0.25) (layer F.Cu) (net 9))
 (segment (start 38.243 33.975) (end 36.091 33.975) (width 0.25) (layer F.Cu) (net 9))
 (segment (start 36.025 37.184) (end 36.052 37.211) (width 0.25) (layer F.Cu) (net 9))
 (segment (start 36.025 33.909) (end 36.025 37.184) (width 0.25) (layer F.Cu) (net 9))
 (segment (start 36.787 53.975) (end 35.433 55.329) (width 0.25) (layer F.Cu) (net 13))
 (segment (start 37.178 53.975) (end 36.787 53.975) (width 0.25) (layer F.Cu) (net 13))
 (segment (start 35.39 43.18) (end 35.136 43.434) (width 0.25) (layer F.Cu) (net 14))
 (segment (start 37.178 43.18) (end 35.39 43.18) (width 0.25) (layer F.Cu) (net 14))
 (segment (start 35.136 43.434) (end 35.136 45.085) (width 0.25) (layer F.Cu) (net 14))
 (segment (start 42.128 52.705) (end 42.578 52.705) (width 0.25) (layer F.Cu) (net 12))
 (segment (start 38.318 48.895) (end 42.128 52.705) (width 0.25) (layer F.Cu) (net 12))
 (segment (start 37.178 48.895) (end 38.318 48.895) (width 0.25) (layer F.Cu) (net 12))
 (segment (start 36.025 48.895) (end 35.306 48.176) (width 0.25) (layer F.Cu) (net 12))
 (segment (start 37.178 48.895) (end 36.025 48.895) (width 0.25) (layer F.Cu) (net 12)))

